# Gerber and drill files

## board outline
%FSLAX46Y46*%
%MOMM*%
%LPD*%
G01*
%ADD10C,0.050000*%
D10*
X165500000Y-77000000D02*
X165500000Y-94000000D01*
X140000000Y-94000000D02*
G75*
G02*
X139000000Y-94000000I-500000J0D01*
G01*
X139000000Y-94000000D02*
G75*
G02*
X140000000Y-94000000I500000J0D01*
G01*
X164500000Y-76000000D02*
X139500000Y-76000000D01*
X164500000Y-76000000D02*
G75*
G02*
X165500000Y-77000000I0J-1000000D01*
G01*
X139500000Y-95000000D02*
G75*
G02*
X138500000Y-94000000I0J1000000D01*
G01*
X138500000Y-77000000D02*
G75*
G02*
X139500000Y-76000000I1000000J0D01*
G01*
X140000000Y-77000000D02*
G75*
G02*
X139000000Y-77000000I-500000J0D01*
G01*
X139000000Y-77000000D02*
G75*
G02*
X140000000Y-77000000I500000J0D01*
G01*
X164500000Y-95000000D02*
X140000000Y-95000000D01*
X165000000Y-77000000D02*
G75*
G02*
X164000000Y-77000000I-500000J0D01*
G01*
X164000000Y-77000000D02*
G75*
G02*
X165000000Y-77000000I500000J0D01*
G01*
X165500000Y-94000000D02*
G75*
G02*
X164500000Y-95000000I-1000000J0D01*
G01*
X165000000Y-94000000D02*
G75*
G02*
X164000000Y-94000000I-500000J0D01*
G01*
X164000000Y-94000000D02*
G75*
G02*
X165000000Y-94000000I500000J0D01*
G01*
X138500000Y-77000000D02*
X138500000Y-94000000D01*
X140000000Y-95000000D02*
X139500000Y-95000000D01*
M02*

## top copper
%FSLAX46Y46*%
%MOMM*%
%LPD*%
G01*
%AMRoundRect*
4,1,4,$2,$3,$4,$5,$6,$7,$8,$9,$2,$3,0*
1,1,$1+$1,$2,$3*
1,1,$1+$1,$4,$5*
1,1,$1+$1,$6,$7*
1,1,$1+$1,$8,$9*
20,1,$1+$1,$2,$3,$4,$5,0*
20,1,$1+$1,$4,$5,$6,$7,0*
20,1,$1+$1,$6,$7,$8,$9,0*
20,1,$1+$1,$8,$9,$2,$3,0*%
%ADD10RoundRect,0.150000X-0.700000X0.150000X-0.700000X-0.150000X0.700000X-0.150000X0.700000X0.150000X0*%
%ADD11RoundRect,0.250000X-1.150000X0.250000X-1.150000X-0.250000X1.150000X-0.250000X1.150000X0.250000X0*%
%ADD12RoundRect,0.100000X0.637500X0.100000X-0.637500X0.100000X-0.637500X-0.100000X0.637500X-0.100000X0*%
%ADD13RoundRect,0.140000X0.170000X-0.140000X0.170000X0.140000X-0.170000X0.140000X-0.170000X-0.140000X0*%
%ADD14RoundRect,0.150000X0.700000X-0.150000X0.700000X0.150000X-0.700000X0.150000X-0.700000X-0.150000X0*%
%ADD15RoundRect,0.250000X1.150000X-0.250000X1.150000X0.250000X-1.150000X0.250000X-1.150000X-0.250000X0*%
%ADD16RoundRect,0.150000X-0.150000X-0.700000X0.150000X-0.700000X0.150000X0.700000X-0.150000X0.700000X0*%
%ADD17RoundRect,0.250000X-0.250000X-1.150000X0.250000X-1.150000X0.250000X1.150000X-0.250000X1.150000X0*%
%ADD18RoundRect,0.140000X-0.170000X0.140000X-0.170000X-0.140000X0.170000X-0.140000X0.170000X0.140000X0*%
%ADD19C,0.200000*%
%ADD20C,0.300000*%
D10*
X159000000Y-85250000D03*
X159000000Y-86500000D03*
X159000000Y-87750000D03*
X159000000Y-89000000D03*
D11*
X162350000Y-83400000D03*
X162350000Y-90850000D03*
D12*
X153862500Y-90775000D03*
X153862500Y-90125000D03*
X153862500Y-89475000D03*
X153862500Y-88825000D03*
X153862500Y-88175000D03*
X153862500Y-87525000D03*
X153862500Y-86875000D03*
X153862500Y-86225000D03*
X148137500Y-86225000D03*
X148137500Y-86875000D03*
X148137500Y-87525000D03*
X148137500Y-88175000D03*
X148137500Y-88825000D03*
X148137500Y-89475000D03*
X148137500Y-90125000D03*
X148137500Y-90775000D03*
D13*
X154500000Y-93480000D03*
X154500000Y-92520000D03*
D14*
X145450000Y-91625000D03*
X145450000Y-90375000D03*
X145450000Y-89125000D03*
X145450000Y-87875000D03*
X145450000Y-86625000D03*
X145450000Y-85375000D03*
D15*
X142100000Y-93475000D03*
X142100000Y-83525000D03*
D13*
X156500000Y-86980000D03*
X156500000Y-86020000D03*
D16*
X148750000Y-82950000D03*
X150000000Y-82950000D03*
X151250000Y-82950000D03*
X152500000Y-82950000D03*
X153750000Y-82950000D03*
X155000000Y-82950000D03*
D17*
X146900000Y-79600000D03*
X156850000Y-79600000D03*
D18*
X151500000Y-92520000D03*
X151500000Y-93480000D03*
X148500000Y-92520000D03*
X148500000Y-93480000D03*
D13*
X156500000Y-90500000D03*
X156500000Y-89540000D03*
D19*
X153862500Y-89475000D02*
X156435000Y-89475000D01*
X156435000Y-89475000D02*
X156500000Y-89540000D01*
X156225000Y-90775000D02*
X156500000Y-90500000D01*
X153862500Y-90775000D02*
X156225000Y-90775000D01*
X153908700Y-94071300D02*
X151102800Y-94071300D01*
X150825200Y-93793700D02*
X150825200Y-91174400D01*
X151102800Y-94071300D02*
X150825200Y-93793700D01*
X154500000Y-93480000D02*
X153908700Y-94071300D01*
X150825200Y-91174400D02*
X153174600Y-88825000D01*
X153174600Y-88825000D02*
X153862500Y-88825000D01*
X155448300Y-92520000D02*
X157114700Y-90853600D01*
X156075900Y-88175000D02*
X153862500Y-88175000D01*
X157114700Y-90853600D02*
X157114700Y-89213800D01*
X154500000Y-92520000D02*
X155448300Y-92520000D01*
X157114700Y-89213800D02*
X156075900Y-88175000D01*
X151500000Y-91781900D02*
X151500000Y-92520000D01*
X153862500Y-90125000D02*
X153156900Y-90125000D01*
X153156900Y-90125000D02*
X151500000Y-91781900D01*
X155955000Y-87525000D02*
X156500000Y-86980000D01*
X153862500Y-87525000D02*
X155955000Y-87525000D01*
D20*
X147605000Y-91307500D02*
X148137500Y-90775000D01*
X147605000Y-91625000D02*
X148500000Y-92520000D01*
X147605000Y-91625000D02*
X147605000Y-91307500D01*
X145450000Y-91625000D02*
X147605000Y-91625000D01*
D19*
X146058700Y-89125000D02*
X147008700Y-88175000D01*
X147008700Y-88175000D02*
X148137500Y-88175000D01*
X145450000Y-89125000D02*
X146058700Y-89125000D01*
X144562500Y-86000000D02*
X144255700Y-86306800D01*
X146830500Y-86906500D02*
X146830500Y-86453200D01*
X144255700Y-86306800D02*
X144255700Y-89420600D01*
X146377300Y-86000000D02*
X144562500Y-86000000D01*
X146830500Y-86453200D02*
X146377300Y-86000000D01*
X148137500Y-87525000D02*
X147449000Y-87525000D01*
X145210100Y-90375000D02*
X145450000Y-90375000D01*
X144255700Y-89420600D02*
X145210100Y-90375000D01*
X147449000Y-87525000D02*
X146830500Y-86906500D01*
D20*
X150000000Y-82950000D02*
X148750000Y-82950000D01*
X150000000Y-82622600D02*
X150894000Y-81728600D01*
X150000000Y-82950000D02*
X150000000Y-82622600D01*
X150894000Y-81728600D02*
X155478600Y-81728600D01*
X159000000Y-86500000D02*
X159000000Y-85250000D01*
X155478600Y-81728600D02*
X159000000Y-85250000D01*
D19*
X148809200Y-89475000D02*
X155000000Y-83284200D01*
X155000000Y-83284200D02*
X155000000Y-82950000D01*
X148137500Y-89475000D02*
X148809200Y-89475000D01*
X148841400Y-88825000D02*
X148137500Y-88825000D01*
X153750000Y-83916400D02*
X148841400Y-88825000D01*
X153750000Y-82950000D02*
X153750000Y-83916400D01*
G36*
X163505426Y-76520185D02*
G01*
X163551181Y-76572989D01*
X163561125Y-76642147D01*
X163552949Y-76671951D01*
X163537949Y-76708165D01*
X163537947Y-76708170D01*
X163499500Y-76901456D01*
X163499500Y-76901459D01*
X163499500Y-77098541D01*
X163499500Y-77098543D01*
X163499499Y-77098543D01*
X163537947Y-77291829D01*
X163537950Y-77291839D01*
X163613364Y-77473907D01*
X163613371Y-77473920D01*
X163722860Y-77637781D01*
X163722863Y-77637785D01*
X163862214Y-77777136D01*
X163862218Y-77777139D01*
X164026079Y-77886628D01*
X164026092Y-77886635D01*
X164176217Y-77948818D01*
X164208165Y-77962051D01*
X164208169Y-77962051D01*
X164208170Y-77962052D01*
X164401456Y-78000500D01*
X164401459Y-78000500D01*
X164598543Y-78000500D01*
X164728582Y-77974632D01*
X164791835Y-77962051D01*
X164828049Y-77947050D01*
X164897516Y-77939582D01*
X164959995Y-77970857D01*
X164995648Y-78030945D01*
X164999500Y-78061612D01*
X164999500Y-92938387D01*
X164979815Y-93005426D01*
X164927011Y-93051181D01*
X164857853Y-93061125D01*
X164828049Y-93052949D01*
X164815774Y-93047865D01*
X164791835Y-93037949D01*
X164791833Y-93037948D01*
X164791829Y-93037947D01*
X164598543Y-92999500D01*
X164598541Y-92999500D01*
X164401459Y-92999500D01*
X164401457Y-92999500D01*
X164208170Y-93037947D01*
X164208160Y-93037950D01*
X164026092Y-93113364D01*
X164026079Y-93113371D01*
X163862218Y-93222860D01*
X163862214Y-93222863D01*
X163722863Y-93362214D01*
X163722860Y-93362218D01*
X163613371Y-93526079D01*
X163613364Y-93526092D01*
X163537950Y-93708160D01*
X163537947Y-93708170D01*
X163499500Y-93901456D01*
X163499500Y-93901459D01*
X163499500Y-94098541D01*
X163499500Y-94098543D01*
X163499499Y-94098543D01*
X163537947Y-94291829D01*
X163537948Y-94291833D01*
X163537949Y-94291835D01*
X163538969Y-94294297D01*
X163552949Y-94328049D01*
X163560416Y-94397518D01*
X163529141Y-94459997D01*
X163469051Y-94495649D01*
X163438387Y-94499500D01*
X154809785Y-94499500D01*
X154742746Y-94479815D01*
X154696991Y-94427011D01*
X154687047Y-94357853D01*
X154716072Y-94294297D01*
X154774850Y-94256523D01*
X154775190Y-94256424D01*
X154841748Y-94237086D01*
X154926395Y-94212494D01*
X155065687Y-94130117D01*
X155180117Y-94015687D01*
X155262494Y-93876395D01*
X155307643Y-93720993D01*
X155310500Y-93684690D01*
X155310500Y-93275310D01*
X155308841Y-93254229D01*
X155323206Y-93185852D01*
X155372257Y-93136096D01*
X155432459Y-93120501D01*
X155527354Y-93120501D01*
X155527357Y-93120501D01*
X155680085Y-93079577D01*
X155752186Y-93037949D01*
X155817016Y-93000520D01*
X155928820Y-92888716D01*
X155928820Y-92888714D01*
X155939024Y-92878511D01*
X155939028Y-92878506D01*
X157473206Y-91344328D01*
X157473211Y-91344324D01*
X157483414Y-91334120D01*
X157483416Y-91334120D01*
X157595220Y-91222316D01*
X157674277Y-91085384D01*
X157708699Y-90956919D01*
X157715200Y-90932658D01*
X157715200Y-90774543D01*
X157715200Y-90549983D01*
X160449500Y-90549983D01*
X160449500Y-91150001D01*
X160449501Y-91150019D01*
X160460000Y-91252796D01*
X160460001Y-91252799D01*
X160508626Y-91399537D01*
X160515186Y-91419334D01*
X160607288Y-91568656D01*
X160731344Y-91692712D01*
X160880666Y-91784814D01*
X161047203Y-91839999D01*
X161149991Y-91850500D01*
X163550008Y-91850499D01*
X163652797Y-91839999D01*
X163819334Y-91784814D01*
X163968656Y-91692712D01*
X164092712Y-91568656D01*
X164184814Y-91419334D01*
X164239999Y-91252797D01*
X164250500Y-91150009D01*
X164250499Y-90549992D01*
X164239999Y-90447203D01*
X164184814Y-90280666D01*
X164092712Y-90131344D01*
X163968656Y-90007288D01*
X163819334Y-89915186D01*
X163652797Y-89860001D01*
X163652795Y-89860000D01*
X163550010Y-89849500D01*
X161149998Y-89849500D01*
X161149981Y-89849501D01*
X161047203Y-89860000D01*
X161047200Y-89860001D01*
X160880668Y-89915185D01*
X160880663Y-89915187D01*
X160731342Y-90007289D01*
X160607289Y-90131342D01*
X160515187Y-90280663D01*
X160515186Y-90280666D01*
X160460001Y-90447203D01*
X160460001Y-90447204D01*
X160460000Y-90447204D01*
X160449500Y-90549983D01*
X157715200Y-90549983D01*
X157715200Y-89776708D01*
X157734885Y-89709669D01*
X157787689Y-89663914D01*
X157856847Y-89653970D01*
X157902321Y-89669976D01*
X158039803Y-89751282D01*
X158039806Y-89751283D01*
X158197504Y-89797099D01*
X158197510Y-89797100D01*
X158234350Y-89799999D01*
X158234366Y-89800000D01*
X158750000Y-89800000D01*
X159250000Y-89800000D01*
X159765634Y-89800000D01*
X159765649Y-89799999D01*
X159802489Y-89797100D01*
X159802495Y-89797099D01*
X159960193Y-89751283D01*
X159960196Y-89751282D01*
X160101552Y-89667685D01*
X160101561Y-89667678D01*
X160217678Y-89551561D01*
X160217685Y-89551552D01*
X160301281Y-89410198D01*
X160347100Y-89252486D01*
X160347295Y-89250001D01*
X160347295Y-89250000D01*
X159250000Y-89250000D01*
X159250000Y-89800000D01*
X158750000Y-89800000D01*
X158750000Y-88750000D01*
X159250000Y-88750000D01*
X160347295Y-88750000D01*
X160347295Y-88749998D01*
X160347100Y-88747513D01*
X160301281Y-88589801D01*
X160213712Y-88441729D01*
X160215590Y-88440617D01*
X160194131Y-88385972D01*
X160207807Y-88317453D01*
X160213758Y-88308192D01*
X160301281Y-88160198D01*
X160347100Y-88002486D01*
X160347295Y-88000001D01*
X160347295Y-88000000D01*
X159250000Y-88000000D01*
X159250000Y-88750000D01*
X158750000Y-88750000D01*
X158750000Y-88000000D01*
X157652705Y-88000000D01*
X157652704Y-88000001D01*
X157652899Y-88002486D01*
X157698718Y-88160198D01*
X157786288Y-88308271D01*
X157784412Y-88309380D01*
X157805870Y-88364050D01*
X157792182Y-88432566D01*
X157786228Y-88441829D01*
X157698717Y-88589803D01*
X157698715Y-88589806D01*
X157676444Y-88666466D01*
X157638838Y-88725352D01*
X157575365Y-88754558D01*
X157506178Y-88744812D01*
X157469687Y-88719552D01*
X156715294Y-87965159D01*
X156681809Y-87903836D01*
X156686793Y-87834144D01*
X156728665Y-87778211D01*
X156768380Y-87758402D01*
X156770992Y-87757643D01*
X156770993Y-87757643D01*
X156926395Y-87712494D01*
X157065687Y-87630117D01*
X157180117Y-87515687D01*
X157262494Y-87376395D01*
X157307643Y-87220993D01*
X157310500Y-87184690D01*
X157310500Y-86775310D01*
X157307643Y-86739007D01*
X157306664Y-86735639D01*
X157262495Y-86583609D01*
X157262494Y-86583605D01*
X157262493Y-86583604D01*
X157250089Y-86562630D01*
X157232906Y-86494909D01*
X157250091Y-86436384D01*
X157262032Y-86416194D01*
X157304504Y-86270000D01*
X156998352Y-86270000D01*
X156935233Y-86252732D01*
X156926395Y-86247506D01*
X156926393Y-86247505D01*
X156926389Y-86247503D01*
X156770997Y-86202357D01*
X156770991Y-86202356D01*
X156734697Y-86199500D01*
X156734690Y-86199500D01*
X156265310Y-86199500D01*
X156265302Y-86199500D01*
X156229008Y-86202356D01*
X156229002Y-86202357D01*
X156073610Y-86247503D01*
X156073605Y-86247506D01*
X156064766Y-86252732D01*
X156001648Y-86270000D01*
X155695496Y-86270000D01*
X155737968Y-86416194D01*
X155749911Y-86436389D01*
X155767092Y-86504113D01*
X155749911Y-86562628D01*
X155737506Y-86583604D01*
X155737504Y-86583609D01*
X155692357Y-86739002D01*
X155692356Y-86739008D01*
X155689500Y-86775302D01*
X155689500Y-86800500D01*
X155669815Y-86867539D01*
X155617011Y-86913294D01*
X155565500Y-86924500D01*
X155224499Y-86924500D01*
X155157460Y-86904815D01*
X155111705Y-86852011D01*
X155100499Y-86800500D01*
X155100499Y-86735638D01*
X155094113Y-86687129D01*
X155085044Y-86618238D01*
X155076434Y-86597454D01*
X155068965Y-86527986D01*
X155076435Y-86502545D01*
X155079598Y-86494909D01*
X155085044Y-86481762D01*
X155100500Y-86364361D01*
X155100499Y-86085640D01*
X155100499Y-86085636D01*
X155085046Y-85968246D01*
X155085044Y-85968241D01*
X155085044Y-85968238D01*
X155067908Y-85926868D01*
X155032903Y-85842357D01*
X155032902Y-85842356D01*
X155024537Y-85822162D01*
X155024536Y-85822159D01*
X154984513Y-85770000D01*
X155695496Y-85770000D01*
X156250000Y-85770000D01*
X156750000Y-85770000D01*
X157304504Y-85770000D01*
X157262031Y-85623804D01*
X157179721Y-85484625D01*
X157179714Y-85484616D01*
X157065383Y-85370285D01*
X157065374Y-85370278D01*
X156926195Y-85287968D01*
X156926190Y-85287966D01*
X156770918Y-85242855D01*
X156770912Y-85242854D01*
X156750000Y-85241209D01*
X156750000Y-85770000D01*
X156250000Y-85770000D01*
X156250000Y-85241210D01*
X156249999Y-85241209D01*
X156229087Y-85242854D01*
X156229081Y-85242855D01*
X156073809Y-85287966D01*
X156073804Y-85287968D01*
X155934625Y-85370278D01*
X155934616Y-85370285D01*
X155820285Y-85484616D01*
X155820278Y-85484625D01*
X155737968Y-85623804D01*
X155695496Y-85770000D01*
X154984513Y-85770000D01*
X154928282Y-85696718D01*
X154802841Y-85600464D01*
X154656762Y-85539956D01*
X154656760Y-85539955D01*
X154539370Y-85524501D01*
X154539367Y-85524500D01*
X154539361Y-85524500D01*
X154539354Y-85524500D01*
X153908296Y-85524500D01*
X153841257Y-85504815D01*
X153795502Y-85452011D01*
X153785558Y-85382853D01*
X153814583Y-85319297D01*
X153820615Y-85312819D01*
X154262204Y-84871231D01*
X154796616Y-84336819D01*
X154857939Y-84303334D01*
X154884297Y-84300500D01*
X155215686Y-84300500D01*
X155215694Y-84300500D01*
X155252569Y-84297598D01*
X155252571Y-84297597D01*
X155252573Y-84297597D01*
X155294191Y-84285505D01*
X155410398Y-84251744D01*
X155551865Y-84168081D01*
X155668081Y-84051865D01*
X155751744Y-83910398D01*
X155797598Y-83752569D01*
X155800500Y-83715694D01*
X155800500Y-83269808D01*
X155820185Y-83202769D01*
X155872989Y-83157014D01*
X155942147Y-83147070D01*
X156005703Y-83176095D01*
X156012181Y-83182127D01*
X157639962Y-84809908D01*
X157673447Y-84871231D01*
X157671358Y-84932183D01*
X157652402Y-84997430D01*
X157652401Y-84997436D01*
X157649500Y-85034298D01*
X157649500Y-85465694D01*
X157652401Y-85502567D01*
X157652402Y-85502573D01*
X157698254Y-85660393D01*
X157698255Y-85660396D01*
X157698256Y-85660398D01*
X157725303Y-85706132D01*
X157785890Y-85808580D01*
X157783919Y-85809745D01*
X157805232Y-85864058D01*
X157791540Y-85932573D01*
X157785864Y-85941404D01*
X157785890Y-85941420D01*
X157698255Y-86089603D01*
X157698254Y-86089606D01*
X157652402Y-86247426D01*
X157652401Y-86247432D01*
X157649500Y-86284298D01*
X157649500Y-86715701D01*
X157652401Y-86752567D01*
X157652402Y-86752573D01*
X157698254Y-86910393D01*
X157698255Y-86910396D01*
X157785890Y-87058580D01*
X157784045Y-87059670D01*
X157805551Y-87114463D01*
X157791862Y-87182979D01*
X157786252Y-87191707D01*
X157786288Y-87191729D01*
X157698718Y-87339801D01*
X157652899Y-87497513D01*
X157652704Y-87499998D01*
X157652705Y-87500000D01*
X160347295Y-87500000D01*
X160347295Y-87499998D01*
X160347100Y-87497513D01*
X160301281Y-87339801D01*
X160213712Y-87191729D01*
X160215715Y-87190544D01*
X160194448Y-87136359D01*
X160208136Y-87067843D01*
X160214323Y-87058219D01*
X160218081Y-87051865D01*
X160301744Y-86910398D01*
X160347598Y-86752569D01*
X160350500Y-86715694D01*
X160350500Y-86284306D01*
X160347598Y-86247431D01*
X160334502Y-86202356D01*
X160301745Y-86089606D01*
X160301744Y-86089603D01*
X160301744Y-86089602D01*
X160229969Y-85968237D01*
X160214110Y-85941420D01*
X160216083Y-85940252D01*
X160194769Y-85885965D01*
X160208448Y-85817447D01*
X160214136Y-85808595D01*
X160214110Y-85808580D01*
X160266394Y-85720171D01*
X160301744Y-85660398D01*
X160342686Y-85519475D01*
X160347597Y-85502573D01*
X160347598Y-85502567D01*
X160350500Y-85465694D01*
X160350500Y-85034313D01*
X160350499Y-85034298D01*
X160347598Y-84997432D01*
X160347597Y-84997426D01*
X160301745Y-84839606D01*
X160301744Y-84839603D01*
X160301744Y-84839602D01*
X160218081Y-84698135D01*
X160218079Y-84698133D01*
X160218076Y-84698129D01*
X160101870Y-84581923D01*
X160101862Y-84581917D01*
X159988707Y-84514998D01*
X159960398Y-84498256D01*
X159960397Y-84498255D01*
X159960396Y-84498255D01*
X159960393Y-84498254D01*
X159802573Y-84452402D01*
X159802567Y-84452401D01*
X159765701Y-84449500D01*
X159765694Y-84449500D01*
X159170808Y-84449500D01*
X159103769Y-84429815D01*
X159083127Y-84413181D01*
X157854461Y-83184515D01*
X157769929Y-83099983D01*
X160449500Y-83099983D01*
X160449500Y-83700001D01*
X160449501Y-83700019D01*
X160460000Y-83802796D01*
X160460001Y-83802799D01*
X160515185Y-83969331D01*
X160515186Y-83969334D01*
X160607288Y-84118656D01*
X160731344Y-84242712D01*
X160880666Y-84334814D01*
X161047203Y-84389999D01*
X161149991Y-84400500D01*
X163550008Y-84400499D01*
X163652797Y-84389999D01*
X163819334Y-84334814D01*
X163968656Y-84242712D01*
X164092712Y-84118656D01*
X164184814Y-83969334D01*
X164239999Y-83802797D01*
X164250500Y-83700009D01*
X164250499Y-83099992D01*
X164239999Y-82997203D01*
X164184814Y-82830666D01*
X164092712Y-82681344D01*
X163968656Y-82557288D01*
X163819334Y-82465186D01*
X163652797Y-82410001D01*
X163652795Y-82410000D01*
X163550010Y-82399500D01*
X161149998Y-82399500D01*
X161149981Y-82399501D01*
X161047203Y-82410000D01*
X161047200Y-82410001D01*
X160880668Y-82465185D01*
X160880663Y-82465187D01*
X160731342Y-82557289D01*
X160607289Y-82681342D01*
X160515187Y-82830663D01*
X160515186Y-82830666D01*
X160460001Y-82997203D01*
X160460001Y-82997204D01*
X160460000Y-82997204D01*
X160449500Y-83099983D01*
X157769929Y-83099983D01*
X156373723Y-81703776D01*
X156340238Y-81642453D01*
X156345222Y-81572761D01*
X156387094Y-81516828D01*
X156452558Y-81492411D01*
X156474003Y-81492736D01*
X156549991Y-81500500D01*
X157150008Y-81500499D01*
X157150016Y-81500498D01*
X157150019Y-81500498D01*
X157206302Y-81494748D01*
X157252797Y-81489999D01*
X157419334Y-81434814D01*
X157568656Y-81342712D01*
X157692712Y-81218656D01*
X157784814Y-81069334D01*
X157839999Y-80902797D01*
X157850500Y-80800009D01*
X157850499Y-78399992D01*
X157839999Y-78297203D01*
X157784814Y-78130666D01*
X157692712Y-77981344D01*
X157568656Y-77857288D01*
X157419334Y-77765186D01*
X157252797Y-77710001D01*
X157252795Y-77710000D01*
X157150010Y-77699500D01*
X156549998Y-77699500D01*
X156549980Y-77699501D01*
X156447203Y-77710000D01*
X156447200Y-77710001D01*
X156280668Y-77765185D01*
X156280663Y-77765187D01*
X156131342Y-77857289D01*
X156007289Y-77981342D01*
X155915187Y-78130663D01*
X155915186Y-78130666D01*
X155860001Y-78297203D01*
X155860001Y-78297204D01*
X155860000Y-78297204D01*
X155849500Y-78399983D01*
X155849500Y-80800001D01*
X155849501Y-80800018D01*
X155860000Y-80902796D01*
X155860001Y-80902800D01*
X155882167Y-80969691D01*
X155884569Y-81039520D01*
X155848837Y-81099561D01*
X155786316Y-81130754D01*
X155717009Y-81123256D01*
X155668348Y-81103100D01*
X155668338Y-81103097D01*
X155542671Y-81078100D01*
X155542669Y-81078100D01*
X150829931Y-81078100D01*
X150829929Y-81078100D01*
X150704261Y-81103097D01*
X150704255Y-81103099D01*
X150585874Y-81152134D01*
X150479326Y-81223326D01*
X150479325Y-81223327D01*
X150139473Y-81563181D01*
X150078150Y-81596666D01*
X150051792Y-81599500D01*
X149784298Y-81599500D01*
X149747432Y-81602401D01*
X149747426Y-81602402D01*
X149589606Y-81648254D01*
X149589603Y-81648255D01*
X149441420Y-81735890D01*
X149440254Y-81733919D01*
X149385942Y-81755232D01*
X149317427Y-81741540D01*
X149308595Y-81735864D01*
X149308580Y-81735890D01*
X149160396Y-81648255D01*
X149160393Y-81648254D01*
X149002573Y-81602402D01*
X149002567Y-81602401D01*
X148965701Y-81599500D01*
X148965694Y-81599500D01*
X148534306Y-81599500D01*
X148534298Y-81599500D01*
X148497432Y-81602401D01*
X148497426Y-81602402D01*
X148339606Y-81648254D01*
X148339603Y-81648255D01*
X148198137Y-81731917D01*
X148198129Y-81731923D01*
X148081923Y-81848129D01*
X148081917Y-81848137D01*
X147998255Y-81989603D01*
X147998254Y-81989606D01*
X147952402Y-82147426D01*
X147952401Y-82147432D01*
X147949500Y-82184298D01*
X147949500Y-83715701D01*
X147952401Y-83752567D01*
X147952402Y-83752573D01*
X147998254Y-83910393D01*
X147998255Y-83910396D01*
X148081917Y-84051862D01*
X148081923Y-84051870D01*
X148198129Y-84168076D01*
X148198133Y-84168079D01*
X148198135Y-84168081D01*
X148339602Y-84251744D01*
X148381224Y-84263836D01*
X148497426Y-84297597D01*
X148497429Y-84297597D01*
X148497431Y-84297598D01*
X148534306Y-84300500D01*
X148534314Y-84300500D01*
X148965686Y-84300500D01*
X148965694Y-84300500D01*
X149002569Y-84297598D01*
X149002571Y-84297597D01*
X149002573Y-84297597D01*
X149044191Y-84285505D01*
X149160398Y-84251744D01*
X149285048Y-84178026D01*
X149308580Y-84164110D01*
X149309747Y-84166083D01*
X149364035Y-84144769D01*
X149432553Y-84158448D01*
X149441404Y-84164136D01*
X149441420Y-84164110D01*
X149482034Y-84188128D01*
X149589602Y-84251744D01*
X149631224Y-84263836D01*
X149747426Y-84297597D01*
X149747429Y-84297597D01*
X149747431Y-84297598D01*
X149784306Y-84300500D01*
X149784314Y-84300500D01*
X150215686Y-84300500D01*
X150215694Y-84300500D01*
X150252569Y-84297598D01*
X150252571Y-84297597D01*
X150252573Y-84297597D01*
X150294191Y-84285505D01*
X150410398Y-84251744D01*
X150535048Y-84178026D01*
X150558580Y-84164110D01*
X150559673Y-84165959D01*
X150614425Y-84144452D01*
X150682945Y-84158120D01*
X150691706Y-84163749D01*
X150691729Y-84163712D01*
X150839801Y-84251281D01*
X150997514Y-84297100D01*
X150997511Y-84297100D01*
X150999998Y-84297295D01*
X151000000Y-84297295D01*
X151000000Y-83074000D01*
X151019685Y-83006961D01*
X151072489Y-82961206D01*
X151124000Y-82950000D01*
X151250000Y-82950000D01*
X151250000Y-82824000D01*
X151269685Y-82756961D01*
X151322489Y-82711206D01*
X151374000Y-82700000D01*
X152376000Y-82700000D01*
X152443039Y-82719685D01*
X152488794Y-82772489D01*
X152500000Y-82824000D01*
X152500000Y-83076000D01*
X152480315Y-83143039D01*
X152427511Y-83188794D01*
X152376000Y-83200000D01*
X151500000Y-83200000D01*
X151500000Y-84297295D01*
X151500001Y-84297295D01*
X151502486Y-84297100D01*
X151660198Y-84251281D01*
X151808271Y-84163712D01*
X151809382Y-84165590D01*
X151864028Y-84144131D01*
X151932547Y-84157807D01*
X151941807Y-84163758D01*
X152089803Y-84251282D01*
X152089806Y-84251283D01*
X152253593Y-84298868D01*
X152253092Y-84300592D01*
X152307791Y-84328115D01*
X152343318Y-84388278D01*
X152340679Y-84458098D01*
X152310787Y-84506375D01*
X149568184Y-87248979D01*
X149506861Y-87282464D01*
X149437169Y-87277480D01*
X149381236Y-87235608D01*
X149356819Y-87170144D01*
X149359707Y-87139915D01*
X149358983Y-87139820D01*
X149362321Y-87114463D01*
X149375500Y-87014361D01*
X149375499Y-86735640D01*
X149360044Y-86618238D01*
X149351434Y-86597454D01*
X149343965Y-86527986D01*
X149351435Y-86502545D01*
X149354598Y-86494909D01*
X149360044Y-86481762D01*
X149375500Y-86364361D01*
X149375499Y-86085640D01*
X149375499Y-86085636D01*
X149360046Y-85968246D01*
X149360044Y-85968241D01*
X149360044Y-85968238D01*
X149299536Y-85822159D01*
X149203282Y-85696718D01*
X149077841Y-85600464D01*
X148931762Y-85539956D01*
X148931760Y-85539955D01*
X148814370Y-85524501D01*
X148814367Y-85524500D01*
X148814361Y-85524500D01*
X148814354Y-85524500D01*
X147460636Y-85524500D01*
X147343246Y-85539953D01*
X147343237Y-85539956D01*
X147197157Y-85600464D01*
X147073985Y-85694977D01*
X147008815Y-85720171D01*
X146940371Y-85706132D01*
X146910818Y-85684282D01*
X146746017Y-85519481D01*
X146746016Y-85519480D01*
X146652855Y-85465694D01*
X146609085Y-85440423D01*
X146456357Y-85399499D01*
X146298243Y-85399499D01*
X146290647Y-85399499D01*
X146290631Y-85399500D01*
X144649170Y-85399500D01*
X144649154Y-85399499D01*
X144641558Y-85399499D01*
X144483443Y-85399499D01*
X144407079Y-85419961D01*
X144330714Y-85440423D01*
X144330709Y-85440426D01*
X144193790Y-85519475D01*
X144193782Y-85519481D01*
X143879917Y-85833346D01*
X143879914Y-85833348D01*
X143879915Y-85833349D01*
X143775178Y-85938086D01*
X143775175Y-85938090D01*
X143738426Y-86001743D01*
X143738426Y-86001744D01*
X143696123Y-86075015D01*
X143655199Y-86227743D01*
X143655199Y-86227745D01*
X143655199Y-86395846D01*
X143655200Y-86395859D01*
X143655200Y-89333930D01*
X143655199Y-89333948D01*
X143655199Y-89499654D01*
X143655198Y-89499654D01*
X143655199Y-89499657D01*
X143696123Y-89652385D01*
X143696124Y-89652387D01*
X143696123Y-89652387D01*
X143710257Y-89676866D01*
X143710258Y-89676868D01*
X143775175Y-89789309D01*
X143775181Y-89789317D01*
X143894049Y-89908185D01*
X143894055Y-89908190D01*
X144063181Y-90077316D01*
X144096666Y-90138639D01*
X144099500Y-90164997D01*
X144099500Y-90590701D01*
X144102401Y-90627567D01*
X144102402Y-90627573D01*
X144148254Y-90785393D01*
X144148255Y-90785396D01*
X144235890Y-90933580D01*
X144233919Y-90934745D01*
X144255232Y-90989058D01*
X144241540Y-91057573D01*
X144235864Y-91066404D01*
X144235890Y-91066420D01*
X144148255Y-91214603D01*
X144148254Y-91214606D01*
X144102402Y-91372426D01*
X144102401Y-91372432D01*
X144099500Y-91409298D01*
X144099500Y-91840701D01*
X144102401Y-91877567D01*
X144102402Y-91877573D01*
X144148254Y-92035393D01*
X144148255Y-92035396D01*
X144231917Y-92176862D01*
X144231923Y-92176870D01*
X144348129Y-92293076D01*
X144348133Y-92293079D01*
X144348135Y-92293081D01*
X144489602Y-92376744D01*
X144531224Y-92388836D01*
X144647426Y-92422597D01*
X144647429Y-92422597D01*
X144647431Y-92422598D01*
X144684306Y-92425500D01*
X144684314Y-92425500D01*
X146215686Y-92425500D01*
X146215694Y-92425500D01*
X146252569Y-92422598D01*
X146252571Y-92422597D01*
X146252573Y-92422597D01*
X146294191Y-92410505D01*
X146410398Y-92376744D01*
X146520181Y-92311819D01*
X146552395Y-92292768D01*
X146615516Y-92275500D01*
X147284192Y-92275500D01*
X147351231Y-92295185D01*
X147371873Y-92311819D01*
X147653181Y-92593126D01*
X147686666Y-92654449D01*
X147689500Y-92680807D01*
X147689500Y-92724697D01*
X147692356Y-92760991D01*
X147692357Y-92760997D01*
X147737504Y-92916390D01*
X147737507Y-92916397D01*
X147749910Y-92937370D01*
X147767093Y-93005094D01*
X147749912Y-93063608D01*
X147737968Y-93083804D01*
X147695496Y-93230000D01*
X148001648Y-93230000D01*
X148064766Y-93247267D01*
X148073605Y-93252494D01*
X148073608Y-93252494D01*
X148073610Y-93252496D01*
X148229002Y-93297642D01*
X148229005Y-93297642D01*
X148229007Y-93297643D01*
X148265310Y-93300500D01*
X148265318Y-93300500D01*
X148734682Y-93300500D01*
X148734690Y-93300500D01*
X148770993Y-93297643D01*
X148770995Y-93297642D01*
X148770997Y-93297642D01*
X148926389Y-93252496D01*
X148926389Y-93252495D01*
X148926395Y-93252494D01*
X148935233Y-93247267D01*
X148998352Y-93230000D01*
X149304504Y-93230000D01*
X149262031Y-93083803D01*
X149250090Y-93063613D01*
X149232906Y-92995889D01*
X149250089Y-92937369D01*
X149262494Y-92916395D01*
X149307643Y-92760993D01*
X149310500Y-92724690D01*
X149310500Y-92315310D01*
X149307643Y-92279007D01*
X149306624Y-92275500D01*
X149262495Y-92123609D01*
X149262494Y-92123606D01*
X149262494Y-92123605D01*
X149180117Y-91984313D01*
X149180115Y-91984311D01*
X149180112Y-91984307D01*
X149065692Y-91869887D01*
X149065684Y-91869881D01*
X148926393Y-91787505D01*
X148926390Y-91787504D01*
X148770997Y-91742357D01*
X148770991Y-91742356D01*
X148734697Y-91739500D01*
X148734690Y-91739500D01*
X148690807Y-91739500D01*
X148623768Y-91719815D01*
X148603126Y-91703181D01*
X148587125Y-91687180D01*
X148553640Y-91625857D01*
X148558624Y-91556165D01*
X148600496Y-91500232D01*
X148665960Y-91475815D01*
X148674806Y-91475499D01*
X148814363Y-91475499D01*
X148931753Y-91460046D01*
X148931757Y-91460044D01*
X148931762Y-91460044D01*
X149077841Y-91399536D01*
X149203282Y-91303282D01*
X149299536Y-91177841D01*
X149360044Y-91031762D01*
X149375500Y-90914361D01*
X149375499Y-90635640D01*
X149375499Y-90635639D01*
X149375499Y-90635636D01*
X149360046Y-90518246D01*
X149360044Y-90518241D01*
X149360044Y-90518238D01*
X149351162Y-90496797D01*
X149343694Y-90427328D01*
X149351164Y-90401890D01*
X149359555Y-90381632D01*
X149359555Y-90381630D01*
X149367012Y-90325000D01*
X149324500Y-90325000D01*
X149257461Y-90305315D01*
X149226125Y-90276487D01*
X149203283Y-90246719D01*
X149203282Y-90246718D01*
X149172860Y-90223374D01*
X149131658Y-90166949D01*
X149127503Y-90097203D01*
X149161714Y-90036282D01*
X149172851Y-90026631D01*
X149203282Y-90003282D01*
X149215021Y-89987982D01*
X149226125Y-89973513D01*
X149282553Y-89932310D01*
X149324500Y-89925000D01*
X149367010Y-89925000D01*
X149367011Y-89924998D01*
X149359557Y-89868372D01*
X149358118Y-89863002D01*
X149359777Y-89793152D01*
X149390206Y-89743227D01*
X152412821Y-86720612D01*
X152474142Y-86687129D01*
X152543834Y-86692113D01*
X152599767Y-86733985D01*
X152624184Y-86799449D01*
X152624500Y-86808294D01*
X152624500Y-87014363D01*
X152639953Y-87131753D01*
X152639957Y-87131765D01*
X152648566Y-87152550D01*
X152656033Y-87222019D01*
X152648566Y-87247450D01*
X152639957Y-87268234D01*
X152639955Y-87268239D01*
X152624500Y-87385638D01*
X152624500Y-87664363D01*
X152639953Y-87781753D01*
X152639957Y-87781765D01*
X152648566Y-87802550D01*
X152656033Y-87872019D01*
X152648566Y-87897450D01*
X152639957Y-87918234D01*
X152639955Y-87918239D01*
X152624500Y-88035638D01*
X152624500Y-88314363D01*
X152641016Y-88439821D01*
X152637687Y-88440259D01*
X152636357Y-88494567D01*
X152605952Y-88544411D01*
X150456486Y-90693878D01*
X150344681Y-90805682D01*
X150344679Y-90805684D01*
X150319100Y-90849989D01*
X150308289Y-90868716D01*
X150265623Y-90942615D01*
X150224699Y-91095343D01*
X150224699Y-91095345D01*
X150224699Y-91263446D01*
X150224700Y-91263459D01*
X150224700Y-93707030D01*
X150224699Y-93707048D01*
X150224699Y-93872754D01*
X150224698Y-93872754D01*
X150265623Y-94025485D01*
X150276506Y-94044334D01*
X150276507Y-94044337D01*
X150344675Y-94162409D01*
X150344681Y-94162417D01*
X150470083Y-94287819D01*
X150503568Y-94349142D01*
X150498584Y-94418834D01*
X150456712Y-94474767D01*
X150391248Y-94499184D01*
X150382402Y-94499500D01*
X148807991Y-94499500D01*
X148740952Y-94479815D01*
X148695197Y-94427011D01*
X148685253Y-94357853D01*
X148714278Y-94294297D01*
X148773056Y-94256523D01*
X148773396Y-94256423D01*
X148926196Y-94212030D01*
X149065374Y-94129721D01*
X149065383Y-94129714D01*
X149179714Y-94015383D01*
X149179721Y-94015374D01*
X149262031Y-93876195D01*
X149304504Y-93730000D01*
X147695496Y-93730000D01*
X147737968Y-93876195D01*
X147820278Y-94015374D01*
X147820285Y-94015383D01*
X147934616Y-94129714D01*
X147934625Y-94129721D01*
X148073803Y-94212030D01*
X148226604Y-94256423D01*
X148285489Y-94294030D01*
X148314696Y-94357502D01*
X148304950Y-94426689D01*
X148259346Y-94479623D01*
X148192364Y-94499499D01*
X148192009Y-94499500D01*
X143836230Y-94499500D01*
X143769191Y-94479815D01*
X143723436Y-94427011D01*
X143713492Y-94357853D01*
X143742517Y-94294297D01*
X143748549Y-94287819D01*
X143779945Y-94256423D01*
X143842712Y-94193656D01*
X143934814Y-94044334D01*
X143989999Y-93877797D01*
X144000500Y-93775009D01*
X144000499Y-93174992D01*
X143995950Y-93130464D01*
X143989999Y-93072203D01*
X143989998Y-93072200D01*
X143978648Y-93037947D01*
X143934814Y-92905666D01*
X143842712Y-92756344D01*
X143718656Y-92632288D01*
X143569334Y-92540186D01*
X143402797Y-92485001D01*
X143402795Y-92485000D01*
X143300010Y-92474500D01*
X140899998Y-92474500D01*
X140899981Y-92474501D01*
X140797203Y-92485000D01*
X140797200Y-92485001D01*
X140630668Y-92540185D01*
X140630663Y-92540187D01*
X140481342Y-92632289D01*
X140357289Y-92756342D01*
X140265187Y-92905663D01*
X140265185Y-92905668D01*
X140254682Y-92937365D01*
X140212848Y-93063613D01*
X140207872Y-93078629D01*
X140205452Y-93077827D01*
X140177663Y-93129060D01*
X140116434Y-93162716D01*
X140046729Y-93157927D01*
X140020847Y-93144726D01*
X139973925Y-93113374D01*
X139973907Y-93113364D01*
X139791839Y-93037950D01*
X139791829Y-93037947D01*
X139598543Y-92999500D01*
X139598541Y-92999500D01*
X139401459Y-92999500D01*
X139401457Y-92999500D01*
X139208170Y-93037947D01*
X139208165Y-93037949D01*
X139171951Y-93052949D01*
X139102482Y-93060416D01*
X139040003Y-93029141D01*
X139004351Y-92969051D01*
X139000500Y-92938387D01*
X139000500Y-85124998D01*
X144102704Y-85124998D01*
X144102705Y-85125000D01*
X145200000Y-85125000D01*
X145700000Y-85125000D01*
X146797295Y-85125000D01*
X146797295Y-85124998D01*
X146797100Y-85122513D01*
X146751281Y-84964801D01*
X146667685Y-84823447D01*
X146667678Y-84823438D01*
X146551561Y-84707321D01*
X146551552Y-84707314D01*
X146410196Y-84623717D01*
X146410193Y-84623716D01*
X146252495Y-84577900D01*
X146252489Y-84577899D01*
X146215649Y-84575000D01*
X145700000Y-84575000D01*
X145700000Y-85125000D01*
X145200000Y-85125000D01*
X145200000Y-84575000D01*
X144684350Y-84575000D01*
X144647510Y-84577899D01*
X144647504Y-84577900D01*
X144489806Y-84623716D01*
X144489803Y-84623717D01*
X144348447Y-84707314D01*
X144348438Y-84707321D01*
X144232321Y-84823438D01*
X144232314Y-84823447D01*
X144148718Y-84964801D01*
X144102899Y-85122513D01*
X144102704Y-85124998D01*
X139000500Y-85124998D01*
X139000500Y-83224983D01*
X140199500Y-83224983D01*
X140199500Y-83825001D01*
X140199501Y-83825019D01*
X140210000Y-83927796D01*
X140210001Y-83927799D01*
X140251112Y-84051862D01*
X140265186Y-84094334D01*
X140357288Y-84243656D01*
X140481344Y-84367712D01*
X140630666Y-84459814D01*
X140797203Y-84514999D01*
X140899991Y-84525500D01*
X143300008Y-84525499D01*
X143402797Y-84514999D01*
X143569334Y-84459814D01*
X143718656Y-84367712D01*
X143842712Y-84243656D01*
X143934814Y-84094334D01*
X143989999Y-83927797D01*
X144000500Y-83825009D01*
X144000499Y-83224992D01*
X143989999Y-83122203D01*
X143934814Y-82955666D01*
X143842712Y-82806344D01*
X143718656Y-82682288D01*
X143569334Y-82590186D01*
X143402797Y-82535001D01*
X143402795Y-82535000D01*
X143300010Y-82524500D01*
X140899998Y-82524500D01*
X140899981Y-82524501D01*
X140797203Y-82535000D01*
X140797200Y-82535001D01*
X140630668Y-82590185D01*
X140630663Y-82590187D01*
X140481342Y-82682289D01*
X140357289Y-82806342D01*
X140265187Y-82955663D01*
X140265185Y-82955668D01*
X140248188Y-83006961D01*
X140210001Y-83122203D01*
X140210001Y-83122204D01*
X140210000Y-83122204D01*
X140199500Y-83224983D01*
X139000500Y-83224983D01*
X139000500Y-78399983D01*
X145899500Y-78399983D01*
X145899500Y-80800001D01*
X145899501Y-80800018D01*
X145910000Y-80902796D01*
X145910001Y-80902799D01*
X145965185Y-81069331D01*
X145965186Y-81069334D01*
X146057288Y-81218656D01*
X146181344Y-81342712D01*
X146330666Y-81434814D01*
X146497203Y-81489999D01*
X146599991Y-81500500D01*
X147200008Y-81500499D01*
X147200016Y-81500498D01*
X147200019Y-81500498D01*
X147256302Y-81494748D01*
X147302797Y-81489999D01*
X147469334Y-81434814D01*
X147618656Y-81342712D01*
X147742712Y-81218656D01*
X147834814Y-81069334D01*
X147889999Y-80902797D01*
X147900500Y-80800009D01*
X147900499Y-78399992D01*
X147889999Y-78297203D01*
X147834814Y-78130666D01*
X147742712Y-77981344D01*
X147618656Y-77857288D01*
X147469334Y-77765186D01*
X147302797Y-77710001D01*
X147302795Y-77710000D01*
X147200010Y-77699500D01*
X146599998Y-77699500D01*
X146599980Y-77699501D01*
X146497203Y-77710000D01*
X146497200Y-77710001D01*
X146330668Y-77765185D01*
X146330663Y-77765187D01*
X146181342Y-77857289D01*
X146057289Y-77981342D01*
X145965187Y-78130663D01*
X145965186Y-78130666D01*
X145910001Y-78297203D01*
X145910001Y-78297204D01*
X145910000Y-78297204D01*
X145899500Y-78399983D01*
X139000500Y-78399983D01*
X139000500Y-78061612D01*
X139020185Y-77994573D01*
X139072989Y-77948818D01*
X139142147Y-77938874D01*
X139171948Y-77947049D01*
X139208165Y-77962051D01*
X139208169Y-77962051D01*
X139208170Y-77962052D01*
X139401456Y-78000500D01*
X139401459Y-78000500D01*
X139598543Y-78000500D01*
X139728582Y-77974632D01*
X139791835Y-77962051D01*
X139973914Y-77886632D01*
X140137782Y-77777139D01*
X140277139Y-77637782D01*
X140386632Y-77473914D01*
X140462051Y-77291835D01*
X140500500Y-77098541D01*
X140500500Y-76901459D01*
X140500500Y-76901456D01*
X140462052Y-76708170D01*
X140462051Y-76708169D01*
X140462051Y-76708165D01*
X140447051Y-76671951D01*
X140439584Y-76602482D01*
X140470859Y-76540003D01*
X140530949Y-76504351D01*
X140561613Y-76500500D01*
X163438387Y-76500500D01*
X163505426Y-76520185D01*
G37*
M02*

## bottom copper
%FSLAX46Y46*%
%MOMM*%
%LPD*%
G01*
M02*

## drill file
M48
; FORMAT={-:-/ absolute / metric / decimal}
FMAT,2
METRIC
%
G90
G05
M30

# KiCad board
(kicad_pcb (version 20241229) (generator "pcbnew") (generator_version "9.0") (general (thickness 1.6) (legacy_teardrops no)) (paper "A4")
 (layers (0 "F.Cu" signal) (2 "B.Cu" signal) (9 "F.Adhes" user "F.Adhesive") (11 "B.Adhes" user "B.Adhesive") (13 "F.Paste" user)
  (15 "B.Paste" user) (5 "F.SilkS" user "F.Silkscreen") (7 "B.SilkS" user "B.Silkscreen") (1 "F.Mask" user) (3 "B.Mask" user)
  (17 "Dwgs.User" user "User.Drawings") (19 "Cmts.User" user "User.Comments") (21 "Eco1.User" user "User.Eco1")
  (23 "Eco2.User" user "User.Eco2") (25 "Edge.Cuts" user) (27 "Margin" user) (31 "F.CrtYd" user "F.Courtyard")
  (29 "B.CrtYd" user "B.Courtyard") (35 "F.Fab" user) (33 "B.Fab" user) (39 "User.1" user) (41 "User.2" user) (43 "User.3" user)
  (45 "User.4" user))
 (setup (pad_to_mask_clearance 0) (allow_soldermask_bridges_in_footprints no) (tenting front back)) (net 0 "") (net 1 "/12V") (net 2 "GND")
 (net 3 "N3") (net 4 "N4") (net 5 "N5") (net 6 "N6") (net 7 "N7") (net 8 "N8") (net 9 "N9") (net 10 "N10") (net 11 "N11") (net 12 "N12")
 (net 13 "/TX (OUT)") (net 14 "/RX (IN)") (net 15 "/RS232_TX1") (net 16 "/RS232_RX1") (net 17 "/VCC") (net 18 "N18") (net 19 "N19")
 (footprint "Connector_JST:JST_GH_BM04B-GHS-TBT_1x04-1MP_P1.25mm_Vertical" (layer "F.Cu") (at 160.95 87.125 -90)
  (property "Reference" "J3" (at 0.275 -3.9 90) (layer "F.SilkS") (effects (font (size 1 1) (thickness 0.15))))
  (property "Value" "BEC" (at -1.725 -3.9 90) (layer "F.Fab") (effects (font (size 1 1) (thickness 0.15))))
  (pad "1" smd roundrect (at -1.875 1.95 270) (size 0.6 1.7) (layers "F.Cu" "F.Mask" "F.Paste") (roundrect_rratio 0.25) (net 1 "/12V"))
  (pad "2" smd roundrect (at -0.625 1.95 270) (size 0.6 1.7) (layers "F.Cu" "F.Mask" "F.Paste") (roundrect_rratio 0.25) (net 1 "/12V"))
  (pad "3" smd roundrect (at 0.625 1.95 270) (size 0.6 1.7) (layers "F.Cu" "F.Mask" "F.Paste") (roundrect_rratio 0.25) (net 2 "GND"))
  (pad "4" smd roundrect (at 1.875 1.95 270) (size 0.6 1.7) (layers "F.Cu" "F.Mask" "F.Paste") (roundrect_rratio 0.25) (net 2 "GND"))
  (pad "MP" smd roundrect (at -3.725 -1.4 270) (size 1 2.8) (layers "F.Cu" "F.Mask" "F.Paste") (roundrect_rratio 0.25))
  (pad "MP" smd roundrect (at 3.725 -1.4 270) (size 1 2.8) (layers "F.Cu" "F.Mask" "F.Paste") (roundrect_rratio 0.25)))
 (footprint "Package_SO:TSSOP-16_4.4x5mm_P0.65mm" (layer "F.Cu") (at 151 88.5 180)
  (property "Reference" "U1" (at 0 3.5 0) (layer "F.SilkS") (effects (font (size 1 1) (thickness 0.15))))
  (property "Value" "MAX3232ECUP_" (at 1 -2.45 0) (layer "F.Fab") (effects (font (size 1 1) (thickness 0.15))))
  (pad "1" smd roundrect (at -2.8625 -2.275 180) (size 1.475 0.4) (layers "F.Cu" "F.Mask" "F.Paste") (roundrect_rratio 0.25) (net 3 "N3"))
  (pad "2" smd roundrect (at -2.8625 -1.625 180) (size 1.475 0.4) (layers "F.Cu" "F.Mask" "F.Paste") (roundrect_rratio 0.25) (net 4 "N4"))
  (pad "3" smd roundrect (at -2.8625 -0.975 180) (size 1.475 0.4) (layers "F.Cu" "F.Mask" "F.Paste") (roundrect_rratio 0.25) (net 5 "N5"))
  (pad "4" smd roundrect (at -2.8625 -0.325 180) (size 1.475 0.4) (layers "F.Cu" "F.Mask" "F.Paste") (roundrect_rratio 0.25) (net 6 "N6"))
  (pad "5" smd roundrect (at -2.8625 0.325 180) (size 1.475 0.4) (layers "F.Cu" "F.Mask" "F.Paste") (roundrect_rratio 0.25) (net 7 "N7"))
  (pad "6" smd roundrect (at -2.8625 0.975 180) (size 1.475 0.4) (layers "F.Cu" "F.Mask" "F.Paste") (roundrect_rratio 0.25) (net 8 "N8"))
  (pad "7" smd roundrect (at -2.8625 1.625 180) (size 1.475 0.4) (layers "F.Cu" "F.Mask" "F.Paste") (roundrect_rratio 0.25) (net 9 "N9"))
  (pad "8" smd roundrect (at -2.8625 2.275 180) (size 1.475 0.4) (layers "F.Cu" "F.Mask" "F.Paste") (roundrect_rratio 0.25) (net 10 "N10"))
  (pad "9" smd roundrect (at 2.8625 2.275 180) (size 1.475 0.4) (layers "F.Cu" "F.Mask" "F.Paste") (roundrect_rratio 0.25) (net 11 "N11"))
  (pad "10" smd roundrect (at 2.8625 1.625 180) (size 1.475 0.4) (layers "F.Cu" "F.Mask" "F.Paste") (roundrect_rratio 0.25) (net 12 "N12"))
  (pad "11" smd roundrect (at 2.8625 0.975 180) (size 1.475 0.4) (layers "F.Cu" "F.Mask" "F.Paste") (roundrect_rratio 0.25)
   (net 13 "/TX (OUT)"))
  (pad "12" smd roundrect (at 2.8625 0.325 180) (size 1.475 0.4) (layers "F.Cu" "F.Mask" "F.Paste") (roundrect_rratio 0.25)
   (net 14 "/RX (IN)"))
  (pad "13" smd roundrect (at 2.8625 -0.325 180) (size 1.475 0.4) (layers "F.Cu" "F.Mask" "F.Paste") (roundrect_rratio 0.25)
   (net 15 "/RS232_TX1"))
  (pad "14" smd roundrect (at 2.8625 -0.975 180) (size 1.475 0.4) (layers "F.Cu" "F.Mask" "F.Paste") (roundrect_rratio 0.25)
   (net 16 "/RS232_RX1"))
  (pad "15" smd roundrect (at 2.8625 -1.625 180) (size 1.475 0.4) (layers "F.Cu" "F.Mask" "F.Paste") (roundrect_rratio 0.25) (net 2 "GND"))
  (pad "16" smd roundrect (at 2.8625 -2.275 180) (size 1.475 0.4) (layers "F.Cu" "F.Mask" "F.Paste") (roundrect_rratio 0.25) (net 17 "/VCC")))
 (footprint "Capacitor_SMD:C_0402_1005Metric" (layer "F.Cu") (at 154.5 93 90)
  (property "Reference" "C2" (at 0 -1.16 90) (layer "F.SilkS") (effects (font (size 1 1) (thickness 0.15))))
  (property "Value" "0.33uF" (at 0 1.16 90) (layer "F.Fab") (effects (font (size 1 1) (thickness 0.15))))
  (pad "1" smd roundrect (at -0.48 0 90) (size 0.56 0.62) (layers "F.Cu" "F.Mask" "F.Paste") (roundrect_rratio 0.25) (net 6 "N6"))
  (pad "2" smd roundrect (at 0.48 0 90) (size 0.56 0.62) (layers "F.Cu" "F.Mask" "F.Paste") (roundrect_rratio 0.25) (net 7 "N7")))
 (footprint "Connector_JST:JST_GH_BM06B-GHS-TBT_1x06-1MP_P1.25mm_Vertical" (layer "F.Cu") (at 143.5 88.5 90)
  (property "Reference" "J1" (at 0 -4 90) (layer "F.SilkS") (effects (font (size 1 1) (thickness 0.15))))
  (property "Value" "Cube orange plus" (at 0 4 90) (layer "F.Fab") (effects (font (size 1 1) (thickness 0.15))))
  (pad "1" smd roundrect (at -3.125 1.95 90) (size 0.6 1.7) (layers "F.Cu" "F.Mask" "F.Paste") (roundrect_rratio 0.25) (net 17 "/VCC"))
  (pad "2" smd roundrect (at -1.875 1.95 90) (size 0.6 1.7) (layers "F.Cu" "F.Mask" "F.Paste") (roundrect_rratio 0.25) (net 13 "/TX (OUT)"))
  (pad "3" smd roundrect (at -0.625 1.95 90) (size 0.6 1.7) (layers "F.Cu" "F.Mask" "F.Paste") (roundrect_rratio 0.25) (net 14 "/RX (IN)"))
  (pad "4" smd roundrect (at 0.625 1.95 90) (size 0.6 1.7) (layers "F.Cu" "F.Mask" "F.Paste") (roundrect_rratio 0.25) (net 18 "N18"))
  (pad "5" smd roundrect (at 1.875 1.95 90) (size 0.6 1.7) (layers "F.Cu" "F.Mask" "F.Paste") (roundrect_rratio 0.25) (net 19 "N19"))
  (pad "6" smd roundrect (at 3.125 1.95 90) (size 0.6 1.7) (layers "F.Cu" "F.Mask" "F.Paste") (roundrect_rratio 0.25) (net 2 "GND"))
  (pad "MP" smd roundrect (at -4.975 -1.4 90) (size 1 2.8) (layers "F.Cu" "F.Mask" "F.Paste") (roundrect_rratio 0.25))
  (pad "MP" smd roundrect (at 4.975 -1.4 90) (size 1 2.8) (layers "F.Cu" "F.Mask" "F.Paste") (roundrect_rratio 0.25)))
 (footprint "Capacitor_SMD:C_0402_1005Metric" (layer "F.Cu") (at 156.5 86.5 90)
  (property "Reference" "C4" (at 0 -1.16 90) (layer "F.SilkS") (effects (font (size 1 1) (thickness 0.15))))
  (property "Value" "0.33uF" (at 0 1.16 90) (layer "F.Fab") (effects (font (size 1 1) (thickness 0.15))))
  (pad "1" smd roundrect (at -0.48 0 90) (size 0.56 0.62) (layers "F.Cu" "F.Mask" "F.Paste") (roundrect_rratio 0.25) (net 8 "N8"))
  (pad "2" smd roundrect (at 0.48 0 90) (size 0.56 0.62) (layers "F.Cu" "F.Mask" "F.Paste") (roundrect_rratio 0.25) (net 2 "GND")))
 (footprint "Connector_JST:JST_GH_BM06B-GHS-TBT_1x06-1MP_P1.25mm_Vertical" (layer "F.Cu") (at 151.875 81)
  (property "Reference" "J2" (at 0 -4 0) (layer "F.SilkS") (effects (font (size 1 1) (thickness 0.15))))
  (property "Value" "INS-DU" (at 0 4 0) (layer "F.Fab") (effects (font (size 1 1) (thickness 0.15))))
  (pad "1" smd roundrect (at -3.125 1.95) (size 0.6 1.7) (layers "F.Cu" "F.Mask" "F.Paste") (roundrect_rratio 0.25) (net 1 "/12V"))
  (pad "2" smd roundrect (at -1.875 1.95) (size 0.6 1.7) (layers "F.Cu" "F.Mask" "F.Paste") (roundrect_rratio 0.25) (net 1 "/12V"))
  (pad "3" smd roundrect (at -0.625 1.95) (size 0.6 1.7) (layers "F.Cu" "F.Mask" "F.Paste") (roundrect_rratio 0.25) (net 2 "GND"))
  (pad "4" smd roundrect (at 0.625 1.95) (size 0.6 1.7) (layers "F.Cu" "F.Mask" "F.Paste") (roundrect_rratio 0.25) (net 2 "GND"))
  (pad "5" smd roundrect (at 1.875 1.95) (size 0.6 1.7) (layers "F.Cu" "F.Mask" "F.Paste") (roundrect_rratio 0.25) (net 15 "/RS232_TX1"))
  (pad "6" smd roundrect (at 3.125 1.95) (size 0.6 1.7) (layers "F.Cu" "F.Mask" "F.Paste") (roundrect_rratio 0.25) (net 16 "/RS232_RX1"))
  (pad "MP" smd roundrect (at -4.975 -1.4) (size 1 2.8) (layers "F.Cu" "F.Mask" "F.Paste") (roundrect_rratio 0.25))
  (pad "MP" smd roundrect (at 4.975 -1.4) (size 1 2.8) (layers "F.Cu" "F.Mask" "F.Paste") (roundrect_rratio 0.25)))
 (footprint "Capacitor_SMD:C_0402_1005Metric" (layer "F.Cu") (at 151.5 93 -90)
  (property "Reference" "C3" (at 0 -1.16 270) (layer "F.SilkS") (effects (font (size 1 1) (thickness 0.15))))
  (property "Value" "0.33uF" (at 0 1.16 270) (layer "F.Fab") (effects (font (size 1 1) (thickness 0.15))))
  (pad "1" smd roundrect (at -0.48 0 270) (size 0.56 0.62) (layers "F.Cu" "F.Mask" "F.Paste") (roundrect_rratio 0.25) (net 4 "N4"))
  (pad "2" smd roundrect (at 0.48 0 270) (size 0.56 0.62) (layers "F.Cu" "F.Mask" "F.Paste") (roundrect_rratio 0.25) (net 2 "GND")))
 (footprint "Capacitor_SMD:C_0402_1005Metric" (layer "F.Cu") (at 148.5 93 -90)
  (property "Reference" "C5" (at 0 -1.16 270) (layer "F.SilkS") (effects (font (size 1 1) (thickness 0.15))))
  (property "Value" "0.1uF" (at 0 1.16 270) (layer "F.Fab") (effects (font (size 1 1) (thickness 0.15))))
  (pad "1" smd roundrect (at -0.48 0 270) (size 0.56 0.62) (layers "F.Cu" "F.Mask" "F.Paste") (roundrect_rratio 0.25) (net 17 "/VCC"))
  (pad "2" smd roundrect (at 0.48 0 270) (size 0.56 0.62) (layers "F.Cu" "F.Mask" "F.Paste") (roundrect_rratio 0.25) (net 2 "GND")))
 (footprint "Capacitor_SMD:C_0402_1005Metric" (layer "F.Cu") (at 156.5 90.02 90)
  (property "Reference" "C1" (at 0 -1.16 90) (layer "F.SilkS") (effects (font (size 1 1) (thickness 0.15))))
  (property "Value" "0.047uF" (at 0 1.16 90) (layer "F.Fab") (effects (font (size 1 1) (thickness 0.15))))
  (pad "1" smd roundrect (at -0.48 0 90) (size 0.56 0.62) (layers "F.Cu" "F.Mask" "F.Paste") (roundrect_rratio 0.25) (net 3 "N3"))
  (pad "2" smd roundrect (at 0.48 0 90) (size 0.56 0.62) (layers "F.Cu" "F.Mask" "F.Paste") (roundrect_rratio 0.25) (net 5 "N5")))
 (gr_line (start 165.5 77) (end 165.5 94) (stroke (width 0.05) (type default)) (layer "Edge.Cuts"))
 (gr_circle (center 139.5 94) (end 139 94) (stroke (width 0.05) (type default)) (fill no) (layer "Edge.Cuts"))
 (gr_line (start 164.5 76) (end 139.5 76) (stroke (width 0.05) (type default)) (layer "Edge.Cuts"))
 (gr_arc (start 164.5 76) (mid 165.207107 76.292893) (end 165.5 77) (stroke (width 0.05) (type default)) (layer "Edge.Cuts"))
 (gr_arc (start 139.5 95) (mid 138.792893 94.707107) (end 138.5 94) (stroke (width 0.05) (type default)) (layer "Edge.Cuts"))
 (gr_arc (start 138.5 77) (mid 138.792893 76.292893) (end 139.5 76) (stroke (width 0.05) (type default)) (layer "Edge.Cuts"))
 (gr_circle (center 139.5 77) (end 139.5 76.5) (stroke (width 0.05) (type default)) (fill no) (layer "Edge.Cuts"))
 (gr_line (start 164.5 95) (end 140 95) (stroke (width 0.05) (type default)) (layer "Edge.Cuts"))
 (gr_circle (center 164.5 77) (end 164.5 77.5) (stroke (width 0.05) (type default)) (fill no) (layer "Edge.Cuts"))
 (gr_arc (start 165.5 94) (mid 165.207107 94.707107) (end 164.5 95) (stroke (width 0.05) (type default)) (layer "Edge.Cuts"))
 (gr_circle (center 164.5 94) (end 165 94) (stroke (width 0.05) (type default)) (fill no) (layer "Edge.Cuts"))
 (gr_line (start 138.5 77) (end 138.5 94) (stroke (width 0.05) (type default)) (layer "Edge.Cuts"))
 (gr_line (start 140 95) (end 139.5 95) (stroke (width 0.05) (type default)) (layer "Edge.Cuts"))
 (segment (start 153.8625 89.475) (end 156.435 89.475) (width 0.2) (layer "F.Cu") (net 5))
 (segment (start 156.435 89.475) (end 156.5 89.54) (width 0.2) (layer "F.Cu") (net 5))
 (segment (start 156.225 90.775) (end 156.5 90.5) (width 0.2) (layer "F.Cu") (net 3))
 (segment (start 153.8625 90.775) (end 156.225 90.775) (width 0.2) (layer "F.Cu") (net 3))
 (segment (start 153.9087 94.0713) (end 151.1028 94.0713) (width 0.2) (layer "F.Cu") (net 6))
 (segment (start 150.8252 93.7937) (end 150.8252 91.1744) (width 0.2) (layer "F.Cu") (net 6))
 (segment (start 151.1028 94.0713) (end 150.8252 93.7937) (width 0.2) (layer "F.Cu") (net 6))
 (segment (start 154.5 93.48) (end 153.9087 94.0713) (width 0.2) (layer "F.Cu") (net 6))
 (segment (start 150.8252 91.1744) (end 153.1746 88.825) (width 0.2) (layer "F.Cu") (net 6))
 (segment (start 153.1746 88.825) (end 153.8625 88.825) (width 0.2) (layer "F.Cu") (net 6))
 (segment (start 155.4483 92.52) (end 157.1147 90.8536) (width 0.2) (layer "F.Cu") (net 7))
 (segment (start 156.0759 88.175) (end 153.8625 88.175) (width 0.2) (layer "F.Cu") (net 7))
 (segment (start 157.1147 90.8536) (end 157.1147 89.2138) (width 0.2) (layer "F.Cu") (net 7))
 (segment (start 154.5 92.52) (end 155.4483 92.52) (width 0.2) (layer "F.Cu") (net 7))
 (segment (start 157.1147 89.2138) (end 156.0759 88.175) (width 0.2) (layer "F.Cu") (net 7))
 (segment (start 151.5 91.7819) (end 151.5 92.52) (width 0.2) (layer "F.Cu") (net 4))
 (segment (start 153.8625 90.125) (end 153.1569 90.125) (width 0.2) (layer "F.Cu") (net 4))
 (segment (start 153.1569 90.125) (end 151.5 91.7819) (width 0.2) (layer "F.Cu") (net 4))
 (segment (start 155.955 87.525) (end 156.5 86.98) (width 0.2) (layer "F.Cu") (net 8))
 (segment (start 153.8625 87.525) (end 155.955 87.525) (width 0.2) (layer "F.Cu") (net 8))
 (segment (start 147.605 91.3075) (end 148.1375 90.775) (width 0.3) (layer "F.Cu") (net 17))
 (segment (start 147.605 91.625) (end 148.5 92.52) (width 0.3) (layer "F.Cu") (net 17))
 (segment (start 147.605 91.625) (end 147.605 91.3075) (width 0.3) (layer "F.Cu") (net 17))
 (segment (start 145.45 91.625) (end 147.605 91.625) (width 0.3) (layer "F.Cu") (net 17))
 (segment (start 146.0587 89.125) (end 147.0087 88.175) (width 0.2) (layer "F.Cu") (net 14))
 (segment (start 147.0087 88.175) (end 148.1375 88.175) (width 0.2) (layer "F.Cu") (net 14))
 (segment (start 145.45 89.125) (end 146.0587 89.125) (width 0.2) (layer "F.Cu") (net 14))
 (segment (start 144.5625 86) (end 144.2557 86.3068) (width 0.2) (layer "F.Cu") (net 13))
 (segment (start 146.8305 86.9065) (end 146.8305 86.4532) (width 0.2) (layer "F.Cu") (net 13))
 (segment (start 144.2557 86.3068) (end 144.2557 89.4206) (width 0.2) (layer "F.Cu") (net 13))
 (segment (start 146.3773 86) (end 144.5625 86) (width 0.2) (layer "F.Cu") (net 13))
 (segment (start 146.8305 86.4532) (end 146.3773 86) (width 0.2) (layer "F.Cu") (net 13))
 (segment (start 148.1375 87.525) (end 147.449 87.525) (width 0.2) (layer "F.Cu") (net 13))
 (segment (start 145.2101 90.375) (end 145.45 90.375) (width 0.2) (layer "F.Cu") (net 13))
 (segment (start 144.2557 89.4206) (end 145.2101 90.375) (width 0.2) (layer "F.Cu") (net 13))
 (segment (start 147.449 87.525) (end 146.8305 86.9065) (width 0.2) (layer "F.Cu") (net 13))
 (segment (start 150 82.95) (end 148.75 82.95) (width 0.3) (layer "F.Cu") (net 1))
 (segment (start 150 82.6226) (end 150.894 81.7286) (width 0.3) (layer "F.Cu") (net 1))
 (segment (start 150 82.95) (end 150 82.6226) (width 0.3) (layer "F.Cu") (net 1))
 (segment (start 150.894 81.7286) (end 155.4786 81.7286) (width 0.3) (layer "F.Cu") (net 1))
 (segment (start 159 86.5) (end 159 85.25) (width 0.3) (layer "F.Cu") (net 1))
 (segment (start 155.4786 81.7286) (end 159 85.25) (width 0.3) (layer "F.Cu") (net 1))
 (segment (start 148.8092 89.475) (end 155 83.2842) (width 0.2) (layer "F.Cu") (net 16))
 (segment (start 155 83.2842) (end 155 82.95) (width 0.2) (layer "F.Cu") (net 16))
 (segment (start 148.1375 89.475) (end 148.8092 89.475) (width 0.2) (layer "F.Cu") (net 16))
 (segment (start 148.8414 88.825) (end 148.1375 88.825) (width 0.2) (layer "F.Cu") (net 15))
 (segment (start 153.75 83.9164) (end 148.8414 88.825) (width 0.2) (layer "F.Cu") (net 15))
 (segment (start 153.75 82.95) (end 153.75 83.9164) (width 0.2) (layer "F.Cu") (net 15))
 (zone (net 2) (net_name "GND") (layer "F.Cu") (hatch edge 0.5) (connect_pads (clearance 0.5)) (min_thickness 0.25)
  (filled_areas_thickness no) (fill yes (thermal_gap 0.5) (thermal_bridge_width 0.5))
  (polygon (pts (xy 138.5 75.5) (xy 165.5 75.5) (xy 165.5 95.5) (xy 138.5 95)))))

